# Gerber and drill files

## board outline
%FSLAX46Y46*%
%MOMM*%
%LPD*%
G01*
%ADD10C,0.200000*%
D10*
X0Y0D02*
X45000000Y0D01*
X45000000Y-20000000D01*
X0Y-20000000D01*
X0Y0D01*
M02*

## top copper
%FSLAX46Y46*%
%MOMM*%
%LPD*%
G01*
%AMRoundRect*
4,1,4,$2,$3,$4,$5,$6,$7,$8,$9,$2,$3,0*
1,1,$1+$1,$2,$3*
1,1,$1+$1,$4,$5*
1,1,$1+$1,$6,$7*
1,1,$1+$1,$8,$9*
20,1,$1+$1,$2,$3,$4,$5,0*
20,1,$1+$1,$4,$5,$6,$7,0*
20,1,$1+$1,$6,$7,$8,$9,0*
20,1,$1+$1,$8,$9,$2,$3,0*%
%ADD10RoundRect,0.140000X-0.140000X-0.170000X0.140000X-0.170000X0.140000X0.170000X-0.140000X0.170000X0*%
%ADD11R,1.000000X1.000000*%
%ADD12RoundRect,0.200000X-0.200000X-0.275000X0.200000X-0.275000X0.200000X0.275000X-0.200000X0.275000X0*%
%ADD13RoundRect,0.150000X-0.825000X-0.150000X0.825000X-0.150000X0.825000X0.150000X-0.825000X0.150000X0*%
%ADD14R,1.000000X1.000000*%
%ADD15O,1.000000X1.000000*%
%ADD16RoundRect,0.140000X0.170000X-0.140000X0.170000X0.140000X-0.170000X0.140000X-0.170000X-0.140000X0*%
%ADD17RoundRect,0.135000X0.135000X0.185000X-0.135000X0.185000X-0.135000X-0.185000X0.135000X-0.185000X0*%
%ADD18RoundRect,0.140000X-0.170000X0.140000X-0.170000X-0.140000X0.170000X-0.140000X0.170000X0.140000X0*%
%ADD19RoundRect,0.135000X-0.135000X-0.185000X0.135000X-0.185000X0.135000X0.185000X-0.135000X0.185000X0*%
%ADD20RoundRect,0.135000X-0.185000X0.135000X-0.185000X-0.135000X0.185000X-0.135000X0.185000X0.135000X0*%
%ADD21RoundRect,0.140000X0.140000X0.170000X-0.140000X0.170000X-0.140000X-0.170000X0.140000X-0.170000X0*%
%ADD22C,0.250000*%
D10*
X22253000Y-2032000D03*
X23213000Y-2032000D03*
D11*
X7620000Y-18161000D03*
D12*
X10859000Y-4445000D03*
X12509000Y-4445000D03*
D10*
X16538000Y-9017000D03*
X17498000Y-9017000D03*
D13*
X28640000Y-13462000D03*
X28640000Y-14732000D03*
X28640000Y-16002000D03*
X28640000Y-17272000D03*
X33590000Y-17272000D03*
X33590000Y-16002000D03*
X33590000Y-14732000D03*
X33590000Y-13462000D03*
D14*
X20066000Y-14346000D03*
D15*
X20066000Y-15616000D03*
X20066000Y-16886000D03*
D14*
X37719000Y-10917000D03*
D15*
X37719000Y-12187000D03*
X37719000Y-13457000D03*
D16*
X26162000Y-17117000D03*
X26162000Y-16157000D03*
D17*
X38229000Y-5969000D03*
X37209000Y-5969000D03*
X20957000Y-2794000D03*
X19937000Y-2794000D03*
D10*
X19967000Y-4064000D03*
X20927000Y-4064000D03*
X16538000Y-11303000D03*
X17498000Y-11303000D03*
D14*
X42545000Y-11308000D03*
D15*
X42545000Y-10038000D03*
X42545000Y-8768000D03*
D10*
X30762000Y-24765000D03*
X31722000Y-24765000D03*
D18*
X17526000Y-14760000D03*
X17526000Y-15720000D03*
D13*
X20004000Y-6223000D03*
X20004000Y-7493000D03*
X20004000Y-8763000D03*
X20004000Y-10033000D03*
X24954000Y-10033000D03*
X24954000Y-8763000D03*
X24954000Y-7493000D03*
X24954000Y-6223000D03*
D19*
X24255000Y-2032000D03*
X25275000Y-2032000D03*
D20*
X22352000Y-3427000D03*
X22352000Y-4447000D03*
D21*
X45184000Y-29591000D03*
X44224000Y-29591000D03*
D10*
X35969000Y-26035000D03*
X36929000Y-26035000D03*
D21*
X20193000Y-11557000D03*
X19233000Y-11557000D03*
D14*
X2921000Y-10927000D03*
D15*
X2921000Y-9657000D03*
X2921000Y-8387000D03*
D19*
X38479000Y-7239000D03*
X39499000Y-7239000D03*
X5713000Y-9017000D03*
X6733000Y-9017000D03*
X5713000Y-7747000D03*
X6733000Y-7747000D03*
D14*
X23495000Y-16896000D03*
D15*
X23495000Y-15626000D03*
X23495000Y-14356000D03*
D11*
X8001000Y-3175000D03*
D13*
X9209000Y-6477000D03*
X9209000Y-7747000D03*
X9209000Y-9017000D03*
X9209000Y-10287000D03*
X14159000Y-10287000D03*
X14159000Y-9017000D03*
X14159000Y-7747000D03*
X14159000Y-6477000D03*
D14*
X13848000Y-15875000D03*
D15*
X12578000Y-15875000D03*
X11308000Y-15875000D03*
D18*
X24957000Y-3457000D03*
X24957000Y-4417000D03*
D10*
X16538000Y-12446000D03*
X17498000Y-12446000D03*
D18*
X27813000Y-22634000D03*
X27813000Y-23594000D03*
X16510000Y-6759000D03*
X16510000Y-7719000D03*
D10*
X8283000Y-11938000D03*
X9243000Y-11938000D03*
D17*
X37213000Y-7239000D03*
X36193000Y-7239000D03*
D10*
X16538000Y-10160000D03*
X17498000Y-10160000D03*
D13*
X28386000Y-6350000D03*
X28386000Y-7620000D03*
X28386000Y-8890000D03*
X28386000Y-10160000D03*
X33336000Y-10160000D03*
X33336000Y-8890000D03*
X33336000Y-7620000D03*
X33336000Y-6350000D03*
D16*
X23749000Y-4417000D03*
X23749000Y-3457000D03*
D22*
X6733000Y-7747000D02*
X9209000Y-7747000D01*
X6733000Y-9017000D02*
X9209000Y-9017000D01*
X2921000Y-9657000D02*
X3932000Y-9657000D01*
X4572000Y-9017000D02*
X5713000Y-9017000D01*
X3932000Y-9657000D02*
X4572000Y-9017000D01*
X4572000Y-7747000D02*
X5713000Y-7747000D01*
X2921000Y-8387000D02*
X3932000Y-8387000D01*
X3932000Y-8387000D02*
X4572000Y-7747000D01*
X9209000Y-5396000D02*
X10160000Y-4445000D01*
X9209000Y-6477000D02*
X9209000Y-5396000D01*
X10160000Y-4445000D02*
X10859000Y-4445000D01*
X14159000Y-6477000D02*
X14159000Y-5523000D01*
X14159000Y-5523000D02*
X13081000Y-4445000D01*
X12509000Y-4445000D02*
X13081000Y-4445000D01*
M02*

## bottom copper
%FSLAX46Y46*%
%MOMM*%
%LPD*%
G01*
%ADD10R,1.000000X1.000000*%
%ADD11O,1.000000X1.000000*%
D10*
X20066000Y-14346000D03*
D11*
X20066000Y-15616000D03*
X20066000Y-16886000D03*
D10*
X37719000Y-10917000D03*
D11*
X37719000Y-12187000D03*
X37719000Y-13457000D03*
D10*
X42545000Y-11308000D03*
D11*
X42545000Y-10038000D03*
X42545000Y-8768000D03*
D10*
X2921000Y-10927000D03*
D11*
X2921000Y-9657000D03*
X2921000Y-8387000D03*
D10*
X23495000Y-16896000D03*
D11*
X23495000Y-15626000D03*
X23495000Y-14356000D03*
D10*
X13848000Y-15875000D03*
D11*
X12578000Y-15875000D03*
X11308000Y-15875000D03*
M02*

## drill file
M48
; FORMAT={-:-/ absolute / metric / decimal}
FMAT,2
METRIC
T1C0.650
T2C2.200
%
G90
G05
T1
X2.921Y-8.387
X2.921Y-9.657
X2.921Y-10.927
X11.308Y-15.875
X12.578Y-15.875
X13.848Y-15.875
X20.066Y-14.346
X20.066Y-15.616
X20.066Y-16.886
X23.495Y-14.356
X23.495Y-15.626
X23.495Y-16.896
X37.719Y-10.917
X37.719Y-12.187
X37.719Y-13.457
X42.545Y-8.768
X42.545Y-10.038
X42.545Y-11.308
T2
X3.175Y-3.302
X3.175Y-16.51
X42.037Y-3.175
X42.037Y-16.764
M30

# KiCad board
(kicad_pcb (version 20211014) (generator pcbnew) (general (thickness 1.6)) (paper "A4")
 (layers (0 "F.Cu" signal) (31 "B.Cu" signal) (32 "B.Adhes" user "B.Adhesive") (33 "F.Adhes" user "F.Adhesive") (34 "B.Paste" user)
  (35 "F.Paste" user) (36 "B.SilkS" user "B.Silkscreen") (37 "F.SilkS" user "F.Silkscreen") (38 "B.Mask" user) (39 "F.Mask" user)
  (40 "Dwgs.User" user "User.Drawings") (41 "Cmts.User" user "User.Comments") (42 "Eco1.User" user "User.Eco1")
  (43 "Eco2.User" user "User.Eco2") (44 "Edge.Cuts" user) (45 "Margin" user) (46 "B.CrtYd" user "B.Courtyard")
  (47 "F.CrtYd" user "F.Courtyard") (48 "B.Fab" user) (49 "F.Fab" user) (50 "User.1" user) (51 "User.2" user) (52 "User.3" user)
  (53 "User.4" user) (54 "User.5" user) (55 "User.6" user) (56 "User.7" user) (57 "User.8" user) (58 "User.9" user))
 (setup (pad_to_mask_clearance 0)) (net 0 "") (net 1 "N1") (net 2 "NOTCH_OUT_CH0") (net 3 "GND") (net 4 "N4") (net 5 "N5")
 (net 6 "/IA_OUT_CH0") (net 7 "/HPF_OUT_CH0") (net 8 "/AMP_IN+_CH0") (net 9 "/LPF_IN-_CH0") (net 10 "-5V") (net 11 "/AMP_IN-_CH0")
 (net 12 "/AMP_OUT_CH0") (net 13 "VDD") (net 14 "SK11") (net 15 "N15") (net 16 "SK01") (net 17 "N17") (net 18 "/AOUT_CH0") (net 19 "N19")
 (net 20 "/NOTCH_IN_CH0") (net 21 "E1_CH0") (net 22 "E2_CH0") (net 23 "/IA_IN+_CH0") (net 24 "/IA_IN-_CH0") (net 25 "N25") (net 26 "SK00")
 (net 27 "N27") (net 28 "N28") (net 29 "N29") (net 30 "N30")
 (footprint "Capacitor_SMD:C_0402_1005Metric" (layer "F.Cu") (at 22.733 2.032)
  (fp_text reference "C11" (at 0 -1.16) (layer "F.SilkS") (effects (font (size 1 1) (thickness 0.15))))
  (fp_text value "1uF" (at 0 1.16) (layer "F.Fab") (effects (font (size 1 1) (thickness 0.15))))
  (pad "1" smd roundrect locked (at -0.48 0) (size 0.56 0.62) (layers "F.Cu" "F.Paste" "F.Mask") (roundrect_rratio 0.25) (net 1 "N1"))
  (pad "2" smd roundrect locked (at 0.48 0) (size 0.56 0.62) (layers "F.Cu" "F.Paste" "F.Mask") (roundrect_rratio 0.25)
   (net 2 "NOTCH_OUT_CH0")))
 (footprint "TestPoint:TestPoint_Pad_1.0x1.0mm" (layer "F.Cu") (at 7.62 18.161)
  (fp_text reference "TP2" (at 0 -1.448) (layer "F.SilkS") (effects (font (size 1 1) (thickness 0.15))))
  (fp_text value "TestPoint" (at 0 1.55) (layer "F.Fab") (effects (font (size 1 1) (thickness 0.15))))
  (pad "1" smd rect locked (at 0 0) (size 1 1) (layers "F.Cu" "F.Mask") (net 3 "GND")))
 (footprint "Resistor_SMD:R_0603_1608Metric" (layer "F.Cu") (at 11.684 4.445)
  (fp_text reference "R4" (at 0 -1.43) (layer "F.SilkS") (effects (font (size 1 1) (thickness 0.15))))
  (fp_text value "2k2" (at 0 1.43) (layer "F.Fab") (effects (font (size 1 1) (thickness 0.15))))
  (pad "1" smd roundrect locked (at -0.825 0) (size 0.8 0.95) (layers "F.Cu" "F.Paste" "F.Mask") (roundrect_rratio 0.25) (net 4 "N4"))
  (pad "2" smd roundrect locked (at 0.825 0) (size 0.8 0.95) (layers "F.Cu" "F.Paste" "F.Mask") (roundrect_rratio 0.25) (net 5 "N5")))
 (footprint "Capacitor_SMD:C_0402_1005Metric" (layer "F.Cu") (at 17.018 9.017)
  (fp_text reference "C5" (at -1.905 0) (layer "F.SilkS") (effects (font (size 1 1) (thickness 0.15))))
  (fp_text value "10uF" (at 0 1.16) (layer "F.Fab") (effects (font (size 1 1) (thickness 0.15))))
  (pad "1" smd roundrect locked (at -0.48 0) (size 0.56 0.62) (layers "F.Cu" "F.Paste" "F.Mask") (roundrect_rratio 0.25)
   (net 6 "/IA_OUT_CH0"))
  (pad "2" smd roundrect locked (at 0.48 0) (size 0.56 0.62) (layers "F.Cu" "F.Paste" "F.Mask") (roundrect_rratio 0.25)
   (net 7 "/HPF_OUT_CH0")))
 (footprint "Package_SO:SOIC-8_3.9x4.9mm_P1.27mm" (layer "F.Cu") (at 31.115 15.367)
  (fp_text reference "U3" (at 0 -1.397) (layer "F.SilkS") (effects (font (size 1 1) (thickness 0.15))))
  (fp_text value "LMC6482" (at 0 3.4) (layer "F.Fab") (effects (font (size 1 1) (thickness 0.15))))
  (pad "1" smd roundrect locked (at -2.475 -1.905) (size 1.95 0.6) (layers "F.Cu" "F.Paste" "F.Mask") (roundrect_rratio 0.25)
   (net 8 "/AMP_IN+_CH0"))
  (pad "2" smd roundrect locked (at -2.475 -0.635) (size 1.95 0.6) (layers "F.Cu" "F.Paste" "F.Mask") (roundrect_rratio 0.25)
   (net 8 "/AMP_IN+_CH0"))
  (pad "3" smd roundrect locked (at -2.475 0.635) (size 1.95 0.6) (layers "F.Cu" "F.Paste" "F.Mask") (roundrect_rratio 0.25)
   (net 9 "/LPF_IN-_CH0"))
  (pad "4" smd roundrect locked (at -2.475 1.905) (size 1.95 0.6) (layers "F.Cu" "F.Paste" "F.Mask") (roundrect_rratio 0.25) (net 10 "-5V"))
  (pad "5" smd roundrect locked (at 2.475 1.905) (size 1.95 0.6) (layers "F.Cu" "F.Paste" "F.Mask") (roundrect_rratio 0.25)
   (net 8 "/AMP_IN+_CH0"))
  (pad "6" smd roundrect locked (at 2.475 0.635) (size 1.95 0.6) (layers "F.Cu" "F.Paste" "F.Mask") (roundrect_rratio 0.25)
   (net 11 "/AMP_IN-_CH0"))
  (pad "7" smd roundrect locked (at 2.475 -0.635) (size 1.95 0.6) (layers "F.Cu" "F.Paste" "F.Mask") (roundrect_rratio 0.25)
   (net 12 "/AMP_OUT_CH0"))
  (pad "8" smd roundrect locked (at 2.475 -1.905) (size 1.95 0.6) (layers "F.Cu" "F.Paste" "F.Mask") (roundrect_rratio 0.25) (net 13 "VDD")))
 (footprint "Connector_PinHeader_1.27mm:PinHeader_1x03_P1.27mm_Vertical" (layer "F.Cu") (at 20.066 14.346)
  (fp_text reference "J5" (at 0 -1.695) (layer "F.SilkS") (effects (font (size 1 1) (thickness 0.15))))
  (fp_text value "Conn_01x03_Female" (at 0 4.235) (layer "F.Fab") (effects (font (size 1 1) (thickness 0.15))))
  (pad "1" thru_hole rect locked (at 0 0) (size 1 1) (drill 0.65) (layers *.Cu *.Mask) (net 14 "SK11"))
  (pad "2" thru_hole oval locked (at 0 1.27) (size 1 1) (drill 0.65) (layers *.Cu *.Mask) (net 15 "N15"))
  (pad "3" thru_hole oval locked (at 0 2.54) (size 1 1) (drill 0.65) (layers *.Cu *.Mask) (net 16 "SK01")))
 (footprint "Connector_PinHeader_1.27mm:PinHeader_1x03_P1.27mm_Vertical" (layer "F.Cu") (at 37.719 10.917)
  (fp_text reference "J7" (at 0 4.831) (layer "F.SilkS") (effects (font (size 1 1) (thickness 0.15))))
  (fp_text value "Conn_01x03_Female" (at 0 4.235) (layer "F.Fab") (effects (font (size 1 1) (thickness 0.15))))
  (pad "1" thru_hole rect locked (at 0 0) (size 1 1) (drill 0.65) (layers *.Cu *.Mask) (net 11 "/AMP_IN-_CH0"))
  (pad "2" thru_hole oval locked (at 0 1.27) (size 1 1) (drill 0.65) (layers *.Cu *.Mask) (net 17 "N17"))
  (pad "3" thru_hole oval locked (at 0 2.54) (size 1 1) (drill 0.65) (layers *.Cu *.Mask) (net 3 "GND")))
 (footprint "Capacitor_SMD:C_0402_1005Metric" (layer "F.Cu") (at 26.162 16.637 90)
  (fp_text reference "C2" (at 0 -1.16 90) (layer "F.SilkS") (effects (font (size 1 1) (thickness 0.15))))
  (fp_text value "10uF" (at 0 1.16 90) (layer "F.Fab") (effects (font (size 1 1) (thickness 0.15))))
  (pad "1" smd roundrect locked (at -0.48 0 90) (size 0.56 0.62) (layers "F.Cu" "F.Paste" "F.Mask") (roundrect_rratio 0.25) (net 16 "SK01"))
  (pad "2" smd roundrect locked (at 0.48 0 90) (size 0.56 0.62) (layers "F.Cu" "F.Paste" "F.Mask") (roundrect_rratio 0.25)
   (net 9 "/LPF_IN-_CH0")))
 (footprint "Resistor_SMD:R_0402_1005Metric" (layer "F.Cu") (at 37.719 5.969 180)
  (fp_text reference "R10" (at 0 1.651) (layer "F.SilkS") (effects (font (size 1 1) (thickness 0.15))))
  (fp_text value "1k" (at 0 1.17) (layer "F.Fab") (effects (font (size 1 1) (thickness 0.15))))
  (pad "1" smd roundrect locked (at -0.51 0 180) (size 0.54 0.64) (layers "F.Cu" "F.Paste" "F.Mask") (roundrect_rratio 0.25)
   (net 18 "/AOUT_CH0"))
  (pad "2" smd roundrect locked (at 0.51 0 180) (size 0.54 0.64) (layers "F.Cu" "F.Paste" "F.Mask") (roundrect_rratio 0.25)
   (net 12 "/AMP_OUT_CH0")))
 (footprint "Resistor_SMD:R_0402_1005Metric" (layer "F.Cu") (at 20.447 2.794 180)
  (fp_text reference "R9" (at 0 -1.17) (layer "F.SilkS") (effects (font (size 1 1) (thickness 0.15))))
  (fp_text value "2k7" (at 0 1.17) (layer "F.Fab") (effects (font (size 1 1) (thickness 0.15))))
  (pad "1" smd roundrect locked (at -0.51 0 180) (size 0.54 0.64) (layers "F.Cu" "F.Paste" "F.Mask") (roundrect_rratio 0.25) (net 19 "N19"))
  (pad "2" smd roundrect locked (at 0.51 0 180) (size 0.54 0.64) (layers "F.Cu" "F.Paste" "F.Mask") (roundrect_rratio 0.25)
   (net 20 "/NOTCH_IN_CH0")))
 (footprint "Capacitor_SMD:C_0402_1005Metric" (layer "F.Cu") (at 20.447 4.064)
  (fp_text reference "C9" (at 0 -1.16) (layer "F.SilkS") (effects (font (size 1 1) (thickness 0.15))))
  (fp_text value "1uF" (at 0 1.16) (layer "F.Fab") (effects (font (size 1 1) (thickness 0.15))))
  (pad "1" smd roundrect locked (at -0.48 0) (size 0.56 0.62) (layers "F.Cu" "F.Paste" "F.Mask") (roundrect_rratio 0.25)
   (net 20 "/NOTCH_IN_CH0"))
  (pad "2" smd roundrect locked (at 0.48 0) (size 0.56 0.62) (layers "F.Cu" "F.Paste" "F.Mask") (roundrect_rratio 0.25) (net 1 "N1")))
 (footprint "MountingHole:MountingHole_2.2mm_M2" (layer "F.Cu") (at 42.037 16.764)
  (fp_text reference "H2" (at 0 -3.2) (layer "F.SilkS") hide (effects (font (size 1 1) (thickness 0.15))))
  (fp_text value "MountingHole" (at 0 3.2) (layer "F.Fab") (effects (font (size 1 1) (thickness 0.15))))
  (pad "" np_thru_hole circle locked (at 0 0) (size 2.2 2.2) (drill 2.2) (layers *.Cu *.Mask)))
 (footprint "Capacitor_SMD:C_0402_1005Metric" (layer "F.Cu") (at 17.018 11.303)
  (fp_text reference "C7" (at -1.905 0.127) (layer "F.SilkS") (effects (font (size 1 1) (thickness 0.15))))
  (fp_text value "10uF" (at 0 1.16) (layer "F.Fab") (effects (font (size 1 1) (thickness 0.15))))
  (pad "1" smd roundrect locked (at -0.48 0) (size 0.56 0.62) (layers "F.Cu" "F.Paste" "F.Mask") (roundrect_rratio 0.25)
   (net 6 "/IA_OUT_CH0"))
  (pad "2" smd roundrect locked (at 0.48 0) (size 0.56 0.62) (layers "F.Cu" "F.Paste" "F.Mask") (roundrect_rratio 0.25)
   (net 7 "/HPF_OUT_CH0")))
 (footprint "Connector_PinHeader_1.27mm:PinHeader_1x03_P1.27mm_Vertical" (layer "F.Cu") (at 42.545 11.308 180)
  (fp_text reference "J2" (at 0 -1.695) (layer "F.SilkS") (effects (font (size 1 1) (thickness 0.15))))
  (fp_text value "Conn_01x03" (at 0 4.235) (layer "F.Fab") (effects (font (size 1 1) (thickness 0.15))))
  (pad "1" thru_hole rect locked (at 0 0 180) (size 1 1) (drill 0.65) (layers *.Cu *.Mask) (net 3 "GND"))
  (pad "2" thru_hole oval locked (at 0 1.27 180) (size 1 1) (drill 0.65) (layers *.Cu *.Mask) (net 18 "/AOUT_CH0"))
  (pad "3" thru_hole oval locked (at 0 2.54 180) (size 1 1) (drill 0.65) (layers *.Cu *.Mask) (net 13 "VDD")))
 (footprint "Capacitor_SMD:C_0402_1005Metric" (layer "F.Cu") (at 31.242 24.765)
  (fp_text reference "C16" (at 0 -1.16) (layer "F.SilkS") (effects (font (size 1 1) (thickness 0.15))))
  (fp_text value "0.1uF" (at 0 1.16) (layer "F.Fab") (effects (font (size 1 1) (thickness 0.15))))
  (pad "1" smd roundrect locked (at -0.48 0) (size 0.56 0.62) (layers "F.Cu" "F.Paste" "F.Mask") (roundrect_rratio 0.25) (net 3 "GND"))
  (pad "2" smd roundrect locked (at 0.48 0) (size 0.56 0.62) (layers "F.Cu" "F.Paste" "F.Mask") (roundrect_rratio 0.25) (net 13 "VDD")))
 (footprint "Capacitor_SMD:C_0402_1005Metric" (layer "F.Cu") (at 17.526 15.24 -90)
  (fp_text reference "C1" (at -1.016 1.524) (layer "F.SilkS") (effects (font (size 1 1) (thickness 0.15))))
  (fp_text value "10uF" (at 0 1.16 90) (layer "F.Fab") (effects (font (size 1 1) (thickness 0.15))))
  (pad "1" smd roundrect locked (at -0.48 0 270) (size 0.56 0.62) (layers "F.Cu" "F.Paste" "F.Mask") (roundrect_rratio 0.25) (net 3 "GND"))
  (pad "2" smd roundrect locked (at 0.48 0 270) (size 0.56 0.62) (layers "F.Cu" "F.Paste" "F.Mask") (roundrect_rratio 0.25) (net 14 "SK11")))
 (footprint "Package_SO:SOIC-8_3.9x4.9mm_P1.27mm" (layer "F.Cu") (at 22.479 8.128)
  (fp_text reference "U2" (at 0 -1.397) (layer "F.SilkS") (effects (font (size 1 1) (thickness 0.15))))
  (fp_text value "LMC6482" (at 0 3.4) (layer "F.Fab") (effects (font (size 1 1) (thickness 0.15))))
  (pad "1" smd roundrect locked (at -2.475 -1.905) (size 1.95 0.6) (layers "F.Cu" "F.Paste" "F.Mask") (roundrect_rratio 0.25)
   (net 20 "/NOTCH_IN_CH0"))
  (pad "2" smd roundrect locked (at -2.475 -0.635) (size 1.95 0.6) (layers "F.Cu" "F.Paste" "F.Mask") (roundrect_rratio 0.25)
   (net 20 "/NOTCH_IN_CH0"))
  (pad "3" smd roundrect locked (at -2.475 0.635) (size 1.95 0.6) (layers "F.Cu" "F.Paste" "F.Mask") (roundrect_rratio 0.25)
   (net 7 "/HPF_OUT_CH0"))
  (pad "4" smd roundrect locked (at -2.475 1.905) (size 1.95 0.6) (layers "F.Cu" "F.Paste" "F.Mask") (roundrect_rratio 0.25) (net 10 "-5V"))
  (pad "5" smd roundrect locked (at 2.475 1.905) (size 1.95 0.6) (layers "F.Cu" "F.Paste" "F.Mask") (roundrect_rratio 0.25) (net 14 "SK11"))
  (pad "6" smd roundrect locked (at 2.475 0.635) (size 1.95 0.6) (layers "F.Cu" "F.Paste" "F.Mask") (roundrect_rratio 0.25)
   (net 9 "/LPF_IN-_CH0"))
  (pad "7" smd roundrect locked (at 2.475 -0.635) (size 1.95 0.6) (layers "F.Cu" "F.Paste" "F.Mask") (roundrect_rratio 0.25)
   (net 9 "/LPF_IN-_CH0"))
  (pad "8" smd roundrect locked (at 2.475 -1.905) (size 1.95 0.6) (layers "F.Cu" "F.Paste" "F.Mask") (roundrect_rratio 0.25) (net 13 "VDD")))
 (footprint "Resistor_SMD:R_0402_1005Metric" (layer "F.Cu") (at 24.765 2.032)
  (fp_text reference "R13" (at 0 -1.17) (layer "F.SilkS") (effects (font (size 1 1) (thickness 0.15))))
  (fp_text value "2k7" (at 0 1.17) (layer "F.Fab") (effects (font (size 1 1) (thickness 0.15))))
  (pad "1" smd roundrect locked (at -0.51 0) (size 0.54 0.64) (layers "F.Cu" "F.Paste" "F.Mask") (roundrect_rratio 0.25)
   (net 2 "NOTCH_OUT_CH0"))
  (pad "2" smd roundrect locked (at 0.51 0) (size 0.54 0.64) (layers "F.Cu" "F.Paste" "F.Mask") (roundrect_rratio 0.25) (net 19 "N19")))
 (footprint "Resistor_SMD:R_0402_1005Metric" (layer "F.Cu") (at 22.352 3.937 -90)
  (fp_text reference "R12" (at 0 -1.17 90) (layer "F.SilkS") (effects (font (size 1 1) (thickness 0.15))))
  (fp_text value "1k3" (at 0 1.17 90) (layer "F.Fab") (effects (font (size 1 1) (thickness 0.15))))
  (pad "1" smd roundrect locked (at -0.51 0 270) (size 0.54 0.64) (layers "F.Cu" "F.Paste" "F.Mask") (roundrect_rratio 0.25) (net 1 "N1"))
  (pad "2" smd roundrect locked (at 0.51 0 270) (size 0.54 0.64) (layers "F.Cu" "F.Paste" "F.Mask") (roundrect_rratio 0.25) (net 3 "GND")))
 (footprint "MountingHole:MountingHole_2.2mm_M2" (layer "F.Cu") (at 3.175 16.51)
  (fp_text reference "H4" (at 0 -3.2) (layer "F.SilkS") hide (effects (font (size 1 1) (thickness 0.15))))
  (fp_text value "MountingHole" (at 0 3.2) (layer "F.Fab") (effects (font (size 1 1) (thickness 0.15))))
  (pad "" np_thru_hole circle locked (at 0 0) (size 2.2 2.2) (drill 2.2) (layers *.Cu *.Mask)))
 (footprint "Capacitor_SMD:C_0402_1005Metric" (layer "F.Cu") (at 44.704 29.591 180)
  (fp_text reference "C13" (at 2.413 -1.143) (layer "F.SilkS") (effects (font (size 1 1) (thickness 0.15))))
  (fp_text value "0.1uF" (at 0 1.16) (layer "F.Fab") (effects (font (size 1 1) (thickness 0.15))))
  (pad "1" smd roundrect locked (at -0.48 0 180) (size 0.56 0.62) (layers "F.Cu" "F.Paste" "F.Mask") (roundrect_rratio 0.25) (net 3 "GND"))
  (pad "2" smd roundrect locked (at 0.48 0 180) (size 0.56 0.62) (layers "F.Cu" "F.Paste" "F.Mask") (roundrect_rratio 0.25) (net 10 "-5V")))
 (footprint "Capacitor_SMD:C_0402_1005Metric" (layer "F.Cu") (at 36.449 26.035)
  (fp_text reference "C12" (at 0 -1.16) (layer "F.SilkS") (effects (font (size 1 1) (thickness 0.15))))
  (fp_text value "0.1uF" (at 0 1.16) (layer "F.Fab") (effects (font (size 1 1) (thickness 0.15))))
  (pad "1" smd roundrect locked (at -0.48 0) (size 0.56 0.62) (layers "F.Cu" "F.Paste" "F.Mask") (roundrect_rratio 0.25) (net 3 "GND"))
  (pad "2" smd roundrect locked (at 0.48 0) (size 0.56 0.62) (layers "F.Cu" "F.Paste" "F.Mask") (roundrect_rratio 0.25) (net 13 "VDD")))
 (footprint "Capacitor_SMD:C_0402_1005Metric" (layer "F.Cu") (at 19.713 11.557 180)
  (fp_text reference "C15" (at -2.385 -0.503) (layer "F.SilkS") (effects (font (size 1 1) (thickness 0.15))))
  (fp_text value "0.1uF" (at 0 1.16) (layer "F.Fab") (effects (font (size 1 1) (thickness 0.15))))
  (pad "1" smd roundrect locked (at -0.48 0 180) (size 0.56 0.62) (layers "F.Cu" "F.Paste" "F.Mask") (roundrect_rratio 0.25) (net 3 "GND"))
  (pad "2" smd roundrect locked (at 0.48 0 180) (size 0.56 0.62) (layers "F.Cu" "F.Paste" "F.Mask") (roundrect_rratio 0.25) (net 10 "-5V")))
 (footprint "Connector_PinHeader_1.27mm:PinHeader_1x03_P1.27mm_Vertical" (layer "F.Cu") (at 2.921 10.927 180)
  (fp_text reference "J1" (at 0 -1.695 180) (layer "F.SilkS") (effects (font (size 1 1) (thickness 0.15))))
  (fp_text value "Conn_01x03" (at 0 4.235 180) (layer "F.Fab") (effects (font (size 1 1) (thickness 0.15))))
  (pad "1" thru_hole rect locked (at 0 0 180) (size 1 1) (drill 0.65) (layers *.Cu *.Mask) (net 3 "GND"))
  (pad "2" thru_hole oval locked (at 0 1.27 180) (size 1 1) (drill 0.65) (layers *.Cu *.Mask) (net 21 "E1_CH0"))
  (pad "3" thru_hole oval locked (at 0 2.54 180) (size 1 1) (drill 0.65) (layers *.Cu *.Mask) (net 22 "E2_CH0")))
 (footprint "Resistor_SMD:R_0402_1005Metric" (layer "F.Cu") (at 38.989 7.239)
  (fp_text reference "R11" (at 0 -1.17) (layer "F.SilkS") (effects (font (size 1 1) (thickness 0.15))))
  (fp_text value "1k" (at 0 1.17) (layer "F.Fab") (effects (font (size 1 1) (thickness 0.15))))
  (pad "1" smd roundrect locked (at -0.51 0) (size 0.54 0.64) (layers "F.Cu" "F.Paste" "F.Mask") (roundrect_rratio 0.25)
   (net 18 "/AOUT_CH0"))
  (pad "2" smd roundrect locked (at 0.51 0) (size 0.54 0.64) (layers "F.Cu" "F.Paste" "F.Mask") (roundrect_rratio 0.25) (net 13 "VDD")))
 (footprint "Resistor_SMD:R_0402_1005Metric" (layer "F.Cu") (at 6.223 9.017)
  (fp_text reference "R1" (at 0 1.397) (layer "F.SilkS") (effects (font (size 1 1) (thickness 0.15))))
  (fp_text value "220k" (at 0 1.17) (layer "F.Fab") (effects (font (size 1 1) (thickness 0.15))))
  (pad "1" smd roundrect locked (at -0.51 0) (size 0.54 0.64) (layers "F.Cu" "F.Paste" "F.Mask") (roundrect_rratio 0.25) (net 21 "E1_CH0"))
  (pad "2" smd roundrect locked (at 0.51 0) (size 0.54 0.64) (layers "F.Cu" "F.Paste" "F.Mask") (roundrect_rratio 0.25)
   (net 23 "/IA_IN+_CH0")))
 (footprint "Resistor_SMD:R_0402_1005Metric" (layer "F.Cu") (at 6.223 7.747)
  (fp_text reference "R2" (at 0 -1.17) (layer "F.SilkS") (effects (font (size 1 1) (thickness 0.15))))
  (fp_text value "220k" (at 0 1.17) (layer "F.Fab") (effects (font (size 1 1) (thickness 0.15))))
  (pad "1" smd roundrect locked (at -0.51 0) (size 0.54 0.64) (layers "F.Cu" "F.Paste" "F.Mask") (roundrect_rratio 0.25) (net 22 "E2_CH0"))
  (pad "2" smd roundrect locked (at 0.51 0) (size 0.54 0.64) (layers "F.Cu" "F.Paste" "F.Mask") (roundrect_rratio 0.25)
   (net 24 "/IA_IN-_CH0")))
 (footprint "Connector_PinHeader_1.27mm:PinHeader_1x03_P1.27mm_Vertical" (layer "F.Cu") (at 23.495 16.896 180)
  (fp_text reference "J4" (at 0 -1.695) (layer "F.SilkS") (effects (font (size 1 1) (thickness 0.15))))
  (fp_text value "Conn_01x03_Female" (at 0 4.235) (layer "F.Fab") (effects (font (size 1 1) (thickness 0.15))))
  (pad "1" thru_hole rect locked (at 0 0 180) (size 1 1) (drill 0.65) (layers *.Cu *.Mask) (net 16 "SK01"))
  (pad "2" thru_hole oval locked (at 0 1.27 180) (size 1 1) (drill 0.65) (layers *.Cu *.Mask) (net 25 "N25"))
  (pad "3" thru_hole oval locked (at 0 2.54 180) (size 1 1) (drill 0.65) (layers *.Cu *.Mask) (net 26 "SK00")))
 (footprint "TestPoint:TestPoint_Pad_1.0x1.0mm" (layer "F.Cu") (at 8.001 3.175)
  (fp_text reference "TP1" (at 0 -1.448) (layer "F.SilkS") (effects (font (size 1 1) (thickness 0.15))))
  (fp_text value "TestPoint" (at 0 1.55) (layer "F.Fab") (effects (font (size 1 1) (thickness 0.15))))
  (pad "1" smd rect locked (at 0 0) (size 1 1) (layers "F.Cu" "F.Mask") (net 3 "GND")))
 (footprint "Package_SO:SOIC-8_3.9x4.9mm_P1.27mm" (layer "F.Cu") (at 11.684 8.382)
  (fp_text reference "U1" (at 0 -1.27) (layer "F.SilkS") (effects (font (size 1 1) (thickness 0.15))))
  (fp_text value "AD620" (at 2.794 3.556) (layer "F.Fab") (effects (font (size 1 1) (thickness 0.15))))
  (pad "1" smd roundrect locked (at -2.475 -1.905) (size 1.95 0.6) (layers "F.Cu" "F.Paste" "F.Mask") (roundrect_rratio 0.25) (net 4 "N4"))
  (pad "2" smd roundrect locked (at -2.475 -0.635) (size 1.95 0.6) (layers "F.Cu" "F.Paste" "F.Mask") (roundrect_rratio 0.25)
   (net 24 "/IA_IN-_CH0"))
  (pad "3" smd roundrect locked (at -2.475 0.635) (size 1.95 0.6) (layers "F.Cu" "F.Paste" "F.Mask") (roundrect_rratio 0.25)
   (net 23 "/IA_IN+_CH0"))
  (pad "4" smd roundrect locked (at -2.475 1.905) (size 1.95 0.6) (layers "F.Cu" "F.Paste" "F.Mask") (roundrect_rratio 0.25) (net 10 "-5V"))
  (pad "5" smd roundrect locked (at 2.475 1.905) (size 1.95 0.6) (layers "F.Cu" "F.Paste" "F.Mask") (roundrect_rratio 0.25) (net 3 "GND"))
  (pad "6" smd roundrect locked (at 2.475 0.635) (size 1.95 0.6) (layers "F.Cu" "F.Paste" "F.Mask") (roundrect_rratio 0.25)
   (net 6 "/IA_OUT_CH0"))
  (pad "7" smd roundrect locked (at 2.475 -0.635) (size 1.95 0.6) (layers "F.Cu" "F.Paste" "F.Mask") (roundrect_rratio 0.25) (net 13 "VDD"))
  (pad "8" smd roundrect locked (at 2.475 -1.905) (size 1.95 0.6) (layers "F.Cu" "F.Paste" "F.Mask") (roundrect_rratio 0.25) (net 5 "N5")))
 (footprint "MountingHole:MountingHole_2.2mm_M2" (layer "F.Cu") (at 3.175 3.302)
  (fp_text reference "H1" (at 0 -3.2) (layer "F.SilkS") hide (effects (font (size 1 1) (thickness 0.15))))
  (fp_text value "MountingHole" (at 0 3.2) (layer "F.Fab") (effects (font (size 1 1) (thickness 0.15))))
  (pad "" np_thru_hole circle locked (at 0 0) (size 2.2 2.2) (drill 2.2) (layers *.Cu *.Mask)))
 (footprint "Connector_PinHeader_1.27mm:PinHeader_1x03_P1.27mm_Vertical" (layer "F.Cu") (at 13.848 15.875 -90)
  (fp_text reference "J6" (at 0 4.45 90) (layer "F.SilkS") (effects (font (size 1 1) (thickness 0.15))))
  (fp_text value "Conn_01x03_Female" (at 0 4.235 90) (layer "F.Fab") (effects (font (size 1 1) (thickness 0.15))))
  (pad "1" thru_hole rect locked (at 0 0 270) (size 1 1) (drill 0.65) (layers *.Cu *.Mask) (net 7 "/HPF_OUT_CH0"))
  (pad "2" thru_hole oval locked (at 0 1.27 270) (size 1 1) (drill 0.65) (layers *.Cu *.Mask) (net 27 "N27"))
  (pad "3" thru_hole oval locked (at 0 2.54 270) (size 1 1) (drill 0.65) (layers *.Cu *.Mask) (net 3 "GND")))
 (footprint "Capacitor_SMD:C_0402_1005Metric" (layer "F.Cu") (at 24.957 3.937 -90)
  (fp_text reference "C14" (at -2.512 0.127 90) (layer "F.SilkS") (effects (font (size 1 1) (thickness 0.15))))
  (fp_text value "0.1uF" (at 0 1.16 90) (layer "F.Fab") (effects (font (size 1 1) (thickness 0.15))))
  (pad "1" smd roundrect locked (at -0.48 0 270) (size 0.56 0.62) (layers "F.Cu" "F.Paste" "F.Mask") (roundrect_rratio 0.25) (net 3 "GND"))
  (pad "2" smd roundrect locked (at 0.48 0 270) (size 0.56 0.62) (layers "F.Cu" "F.Paste" "F.Mask") (roundrect_rratio 0.25) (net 13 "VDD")))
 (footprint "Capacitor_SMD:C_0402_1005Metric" (layer "F.Cu") (at 17.018 12.446)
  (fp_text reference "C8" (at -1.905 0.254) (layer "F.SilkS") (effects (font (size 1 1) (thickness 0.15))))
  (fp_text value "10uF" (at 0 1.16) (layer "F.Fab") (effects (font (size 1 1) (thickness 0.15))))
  (pad "1" smd roundrect locked (at -0.48 0) (size 0.56 0.62) (layers "F.Cu" "F.Paste" "F.Mask") (roundrect_rratio 0.25)
   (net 6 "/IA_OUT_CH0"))
  (pad "2" smd roundrect locked (at 0.48 0) (size 0.56 0.62) (layers "F.Cu" "F.Paste" "F.Mask") (roundrect_rratio 0.25)
   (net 7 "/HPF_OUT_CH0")))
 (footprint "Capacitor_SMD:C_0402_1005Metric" (layer "F.Cu") (at 27.813 23.114 -90)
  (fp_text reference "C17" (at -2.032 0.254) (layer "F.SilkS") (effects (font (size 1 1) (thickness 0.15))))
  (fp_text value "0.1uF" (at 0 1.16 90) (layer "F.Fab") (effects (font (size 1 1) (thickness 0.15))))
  (pad "1" smd roundrect locked (at -0.48 0 270) (size 0.56 0.62) (layers "F.Cu" "F.Paste" "F.Mask") (roundrect_rratio 0.25) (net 3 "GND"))
  (pad "2" smd roundrect locked (at 0.48 0 270) (size 0.56 0.62) (layers "F.Cu" "F.Paste" "F.Mask") (roundrect_rratio 0.25) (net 10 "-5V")))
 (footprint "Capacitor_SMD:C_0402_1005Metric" (layer "F.Cu") (at 16.51 7.239 -90)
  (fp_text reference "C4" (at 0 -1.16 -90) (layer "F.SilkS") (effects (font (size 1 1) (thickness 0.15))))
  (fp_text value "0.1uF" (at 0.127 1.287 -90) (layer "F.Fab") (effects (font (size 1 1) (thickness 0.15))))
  (pad "1" smd roundrect locked (at -0.48 0 270) (size 0.56 0.62) (layers "F.Cu" "F.Paste" "F.Mask") (roundrect_rratio 0.25) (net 3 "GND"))
  (pad "2" smd roundrect locked (at 0.48 0 270) (size 0.56 0.62) (layers "F.Cu" "F.Paste" "F.Mask") (roundrect_rratio 0.25) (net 13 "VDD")))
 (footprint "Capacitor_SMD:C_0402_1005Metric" (layer "F.Cu") (at 8.763 11.938)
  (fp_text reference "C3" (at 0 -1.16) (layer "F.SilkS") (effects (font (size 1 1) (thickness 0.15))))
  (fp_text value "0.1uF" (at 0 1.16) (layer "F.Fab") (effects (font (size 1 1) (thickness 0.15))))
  (pad "1" smd roundrect locked (at -0.48 0) (size 0.56 0.62) (layers "F.Cu" "F.Paste" "F.Mask") (roundrect_rratio 0.25) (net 3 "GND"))
  (pad "2" smd roundrect locked (at 0.48 0) (size 0.56 0.62) (layers "F.Cu" "F.Paste" "F.Mask") (roundrect_rratio 0.25) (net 10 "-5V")))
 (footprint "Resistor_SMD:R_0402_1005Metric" (layer "F.Cu") (at 36.703 7.239 180)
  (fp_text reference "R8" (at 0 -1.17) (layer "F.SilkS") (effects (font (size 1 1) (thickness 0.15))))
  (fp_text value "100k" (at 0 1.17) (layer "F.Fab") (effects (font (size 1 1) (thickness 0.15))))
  (pad "1" smd roundrect locked (at -0.51 0 180) (size 0.54 0.64) (layers "F.Cu" "F.Paste" "F.Mask") (roundrect_rratio 0.25)
   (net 12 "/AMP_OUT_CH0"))
  (pad "2" smd roundrect locked (at 0.51 0 180) (size 0.54 0.64) (layers "F.Cu" "F.Paste" "F.Mask") (roundrect_rratio 0.25)
   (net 11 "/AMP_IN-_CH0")))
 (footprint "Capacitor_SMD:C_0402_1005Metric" (layer "F.Cu") (at 17.018 10.16)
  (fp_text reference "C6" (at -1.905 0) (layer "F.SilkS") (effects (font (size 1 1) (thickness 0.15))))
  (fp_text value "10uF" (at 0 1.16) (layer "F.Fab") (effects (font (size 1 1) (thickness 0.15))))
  (pad "1" smd roundrect locked (at -0.48 0) (size 0.56 0.62) (layers "F.Cu" "F.Paste" "F.Mask") (roundrect_rratio 0.25)
   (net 6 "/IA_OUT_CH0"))
  (pad "2" smd roundrect locked (at 0.48 0) (size 0.56 0.62) (layers "F.Cu" "F.Paste" "F.Mask") (roundrect_rratio 0.25)
   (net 7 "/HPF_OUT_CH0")))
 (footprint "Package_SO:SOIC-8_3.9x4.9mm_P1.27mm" (layer "F.Cu") (at 30.861 8.255)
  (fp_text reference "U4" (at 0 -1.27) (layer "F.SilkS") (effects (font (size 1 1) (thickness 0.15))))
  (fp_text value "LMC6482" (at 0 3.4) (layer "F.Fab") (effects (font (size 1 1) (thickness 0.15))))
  (pad "1" smd roundrect locked (at -2.475 -1.905) (size 1.95 0.6) (layers "F.Cu" "F.Paste" "F.Mask") (roundrect_rratio 0.25)
   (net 26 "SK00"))
  (pad "2" smd roundrect locked (at -2.475 -0.635) (size 1.95 0.6) (layers "F.Cu" "F.Paste" "F.Mask") (roundrect_rratio 0.25)
   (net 26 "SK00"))
  (pad "3" smd roundrect locked (at -2.475 0.635) (size 1.95 0.6) (layers "F.Cu" "F.Paste" "F.Mask") (roundrect_rratio 0.25)
   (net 2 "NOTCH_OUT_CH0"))
  (pad "4" smd roundrect locked (at -2.475 1.905) (size 1.95 0.6) (layers "F.Cu" "F.Paste" "F.Mask") (roundrect_rratio 0.25) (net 10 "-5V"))
  (pad "5" smd roundrect locked (at 2.475 1.905) (size 1.95 0.6) (layers "F.Cu" "F.Paste" "F.Mask") (roundrect_rratio 0.25) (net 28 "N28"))
  (pad "6" smd roundrect locked (at 2.475 0.635) (size 1.95 0.6) (layers "F.Cu" "F.Paste" "F.Mask") (roundrect_rratio 0.25) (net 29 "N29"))
  (pad "7" smd roundrect locked (at 2.475 -0.635) (size 1.95 0.6) (layers "F.Cu" "F.Paste" "F.Mask") (roundrect_rratio 0.25) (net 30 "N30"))
  (pad "8" smd roundrect locked (at 2.475 -1.905) (size 1.95 0.6) (layers "F.Cu" "F.Paste" "F.Mask") (roundrect_rratio 0.25) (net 13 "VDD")))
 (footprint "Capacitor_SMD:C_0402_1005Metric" (layer "F.Cu") (at 23.749 3.937 90)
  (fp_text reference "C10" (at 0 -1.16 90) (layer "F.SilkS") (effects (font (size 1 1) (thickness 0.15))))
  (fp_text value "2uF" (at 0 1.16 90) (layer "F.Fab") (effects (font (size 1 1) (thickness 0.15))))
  (pad "1" smd roundrect locked (at -0.48 0 90) (size 0.56 0.62) (layers "F.Cu" "F.Paste" "F.Mask") (roundrect_rratio 0.25) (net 3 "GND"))
  (pad "2" smd roundrect locked (at 0.48 0 90) (size 0.56 0.62) (layers "F.Cu" "F.Paste" "F.Mask") (roundrect_rratio 0.25) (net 19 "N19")))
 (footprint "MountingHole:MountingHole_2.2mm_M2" (layer "F.Cu") (at 42.037 3.175)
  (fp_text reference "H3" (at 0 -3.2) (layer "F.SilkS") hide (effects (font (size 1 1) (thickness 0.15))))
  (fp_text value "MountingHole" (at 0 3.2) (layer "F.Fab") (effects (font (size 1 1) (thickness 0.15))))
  (pad "" np_thru_hole circle locked (at 0 0) (size 2.2 2.2) (drill 2.2) (layers *.Cu *.Mask)))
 (gr_rect (start 0 0) (end 45 20) (layer "Edge.Cuts") (width 0.2) (fill none))
 (segment (start 6.733 7.747) (end 9.209 7.747) (width 0.25) (layer "F.Cu") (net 24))
 (segment (start 6.733 9.017) (end 9.209 9.017) (width 0.25) (layer "F.Cu") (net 23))
 (segment (start 2.921 9.657) (end 3.932 9.657) (width 0.25) (layer "F.Cu") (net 21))
 (segment (start 4.572 9.017) (end 5.713 9.017) (width 0.25) (layer "F.Cu") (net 21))
 (segment (start 3.932 9.657) (end 4.572 9.017) (width 0.25) (layer "F.Cu") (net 21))
 (segment (start 4.572 7.747) (end 5.713 7.747) (width 0.25) (layer "F.Cu") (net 22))
 (segment (start 2.921 8.387) (end 3.932 8.387) (width 0.25) (layer "F.Cu") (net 22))
 (segment (start 3.932 8.387) (end 4.572 7.747) (width 0.25) (layer "F.Cu") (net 22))
 (segment (start 9.209 5.396) (end 10.16 4.445) (width 0.25) (layer "F.Cu") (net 4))
 (segment (start 9.209 6.477) (end 9.209 5.396) (width 0.25) (layer "F.Cu") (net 4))
 (segment (start 10.16 4.445) (end 10.859 4.445) (width 0.25) (layer "F.Cu") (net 4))
 (segment (start 14.159 6.477) (end 14.159 5.523) (width 0.25) (layer "F.Cu") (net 5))
 (segment (start 14.159 5.523) (end 13.081 4.445) (width 0.25) (layer "F.Cu") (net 5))
 (segment (start 12.509 4.445) (end 13.081 4.445) (width 0.25) (layer "F.Cu") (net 5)))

